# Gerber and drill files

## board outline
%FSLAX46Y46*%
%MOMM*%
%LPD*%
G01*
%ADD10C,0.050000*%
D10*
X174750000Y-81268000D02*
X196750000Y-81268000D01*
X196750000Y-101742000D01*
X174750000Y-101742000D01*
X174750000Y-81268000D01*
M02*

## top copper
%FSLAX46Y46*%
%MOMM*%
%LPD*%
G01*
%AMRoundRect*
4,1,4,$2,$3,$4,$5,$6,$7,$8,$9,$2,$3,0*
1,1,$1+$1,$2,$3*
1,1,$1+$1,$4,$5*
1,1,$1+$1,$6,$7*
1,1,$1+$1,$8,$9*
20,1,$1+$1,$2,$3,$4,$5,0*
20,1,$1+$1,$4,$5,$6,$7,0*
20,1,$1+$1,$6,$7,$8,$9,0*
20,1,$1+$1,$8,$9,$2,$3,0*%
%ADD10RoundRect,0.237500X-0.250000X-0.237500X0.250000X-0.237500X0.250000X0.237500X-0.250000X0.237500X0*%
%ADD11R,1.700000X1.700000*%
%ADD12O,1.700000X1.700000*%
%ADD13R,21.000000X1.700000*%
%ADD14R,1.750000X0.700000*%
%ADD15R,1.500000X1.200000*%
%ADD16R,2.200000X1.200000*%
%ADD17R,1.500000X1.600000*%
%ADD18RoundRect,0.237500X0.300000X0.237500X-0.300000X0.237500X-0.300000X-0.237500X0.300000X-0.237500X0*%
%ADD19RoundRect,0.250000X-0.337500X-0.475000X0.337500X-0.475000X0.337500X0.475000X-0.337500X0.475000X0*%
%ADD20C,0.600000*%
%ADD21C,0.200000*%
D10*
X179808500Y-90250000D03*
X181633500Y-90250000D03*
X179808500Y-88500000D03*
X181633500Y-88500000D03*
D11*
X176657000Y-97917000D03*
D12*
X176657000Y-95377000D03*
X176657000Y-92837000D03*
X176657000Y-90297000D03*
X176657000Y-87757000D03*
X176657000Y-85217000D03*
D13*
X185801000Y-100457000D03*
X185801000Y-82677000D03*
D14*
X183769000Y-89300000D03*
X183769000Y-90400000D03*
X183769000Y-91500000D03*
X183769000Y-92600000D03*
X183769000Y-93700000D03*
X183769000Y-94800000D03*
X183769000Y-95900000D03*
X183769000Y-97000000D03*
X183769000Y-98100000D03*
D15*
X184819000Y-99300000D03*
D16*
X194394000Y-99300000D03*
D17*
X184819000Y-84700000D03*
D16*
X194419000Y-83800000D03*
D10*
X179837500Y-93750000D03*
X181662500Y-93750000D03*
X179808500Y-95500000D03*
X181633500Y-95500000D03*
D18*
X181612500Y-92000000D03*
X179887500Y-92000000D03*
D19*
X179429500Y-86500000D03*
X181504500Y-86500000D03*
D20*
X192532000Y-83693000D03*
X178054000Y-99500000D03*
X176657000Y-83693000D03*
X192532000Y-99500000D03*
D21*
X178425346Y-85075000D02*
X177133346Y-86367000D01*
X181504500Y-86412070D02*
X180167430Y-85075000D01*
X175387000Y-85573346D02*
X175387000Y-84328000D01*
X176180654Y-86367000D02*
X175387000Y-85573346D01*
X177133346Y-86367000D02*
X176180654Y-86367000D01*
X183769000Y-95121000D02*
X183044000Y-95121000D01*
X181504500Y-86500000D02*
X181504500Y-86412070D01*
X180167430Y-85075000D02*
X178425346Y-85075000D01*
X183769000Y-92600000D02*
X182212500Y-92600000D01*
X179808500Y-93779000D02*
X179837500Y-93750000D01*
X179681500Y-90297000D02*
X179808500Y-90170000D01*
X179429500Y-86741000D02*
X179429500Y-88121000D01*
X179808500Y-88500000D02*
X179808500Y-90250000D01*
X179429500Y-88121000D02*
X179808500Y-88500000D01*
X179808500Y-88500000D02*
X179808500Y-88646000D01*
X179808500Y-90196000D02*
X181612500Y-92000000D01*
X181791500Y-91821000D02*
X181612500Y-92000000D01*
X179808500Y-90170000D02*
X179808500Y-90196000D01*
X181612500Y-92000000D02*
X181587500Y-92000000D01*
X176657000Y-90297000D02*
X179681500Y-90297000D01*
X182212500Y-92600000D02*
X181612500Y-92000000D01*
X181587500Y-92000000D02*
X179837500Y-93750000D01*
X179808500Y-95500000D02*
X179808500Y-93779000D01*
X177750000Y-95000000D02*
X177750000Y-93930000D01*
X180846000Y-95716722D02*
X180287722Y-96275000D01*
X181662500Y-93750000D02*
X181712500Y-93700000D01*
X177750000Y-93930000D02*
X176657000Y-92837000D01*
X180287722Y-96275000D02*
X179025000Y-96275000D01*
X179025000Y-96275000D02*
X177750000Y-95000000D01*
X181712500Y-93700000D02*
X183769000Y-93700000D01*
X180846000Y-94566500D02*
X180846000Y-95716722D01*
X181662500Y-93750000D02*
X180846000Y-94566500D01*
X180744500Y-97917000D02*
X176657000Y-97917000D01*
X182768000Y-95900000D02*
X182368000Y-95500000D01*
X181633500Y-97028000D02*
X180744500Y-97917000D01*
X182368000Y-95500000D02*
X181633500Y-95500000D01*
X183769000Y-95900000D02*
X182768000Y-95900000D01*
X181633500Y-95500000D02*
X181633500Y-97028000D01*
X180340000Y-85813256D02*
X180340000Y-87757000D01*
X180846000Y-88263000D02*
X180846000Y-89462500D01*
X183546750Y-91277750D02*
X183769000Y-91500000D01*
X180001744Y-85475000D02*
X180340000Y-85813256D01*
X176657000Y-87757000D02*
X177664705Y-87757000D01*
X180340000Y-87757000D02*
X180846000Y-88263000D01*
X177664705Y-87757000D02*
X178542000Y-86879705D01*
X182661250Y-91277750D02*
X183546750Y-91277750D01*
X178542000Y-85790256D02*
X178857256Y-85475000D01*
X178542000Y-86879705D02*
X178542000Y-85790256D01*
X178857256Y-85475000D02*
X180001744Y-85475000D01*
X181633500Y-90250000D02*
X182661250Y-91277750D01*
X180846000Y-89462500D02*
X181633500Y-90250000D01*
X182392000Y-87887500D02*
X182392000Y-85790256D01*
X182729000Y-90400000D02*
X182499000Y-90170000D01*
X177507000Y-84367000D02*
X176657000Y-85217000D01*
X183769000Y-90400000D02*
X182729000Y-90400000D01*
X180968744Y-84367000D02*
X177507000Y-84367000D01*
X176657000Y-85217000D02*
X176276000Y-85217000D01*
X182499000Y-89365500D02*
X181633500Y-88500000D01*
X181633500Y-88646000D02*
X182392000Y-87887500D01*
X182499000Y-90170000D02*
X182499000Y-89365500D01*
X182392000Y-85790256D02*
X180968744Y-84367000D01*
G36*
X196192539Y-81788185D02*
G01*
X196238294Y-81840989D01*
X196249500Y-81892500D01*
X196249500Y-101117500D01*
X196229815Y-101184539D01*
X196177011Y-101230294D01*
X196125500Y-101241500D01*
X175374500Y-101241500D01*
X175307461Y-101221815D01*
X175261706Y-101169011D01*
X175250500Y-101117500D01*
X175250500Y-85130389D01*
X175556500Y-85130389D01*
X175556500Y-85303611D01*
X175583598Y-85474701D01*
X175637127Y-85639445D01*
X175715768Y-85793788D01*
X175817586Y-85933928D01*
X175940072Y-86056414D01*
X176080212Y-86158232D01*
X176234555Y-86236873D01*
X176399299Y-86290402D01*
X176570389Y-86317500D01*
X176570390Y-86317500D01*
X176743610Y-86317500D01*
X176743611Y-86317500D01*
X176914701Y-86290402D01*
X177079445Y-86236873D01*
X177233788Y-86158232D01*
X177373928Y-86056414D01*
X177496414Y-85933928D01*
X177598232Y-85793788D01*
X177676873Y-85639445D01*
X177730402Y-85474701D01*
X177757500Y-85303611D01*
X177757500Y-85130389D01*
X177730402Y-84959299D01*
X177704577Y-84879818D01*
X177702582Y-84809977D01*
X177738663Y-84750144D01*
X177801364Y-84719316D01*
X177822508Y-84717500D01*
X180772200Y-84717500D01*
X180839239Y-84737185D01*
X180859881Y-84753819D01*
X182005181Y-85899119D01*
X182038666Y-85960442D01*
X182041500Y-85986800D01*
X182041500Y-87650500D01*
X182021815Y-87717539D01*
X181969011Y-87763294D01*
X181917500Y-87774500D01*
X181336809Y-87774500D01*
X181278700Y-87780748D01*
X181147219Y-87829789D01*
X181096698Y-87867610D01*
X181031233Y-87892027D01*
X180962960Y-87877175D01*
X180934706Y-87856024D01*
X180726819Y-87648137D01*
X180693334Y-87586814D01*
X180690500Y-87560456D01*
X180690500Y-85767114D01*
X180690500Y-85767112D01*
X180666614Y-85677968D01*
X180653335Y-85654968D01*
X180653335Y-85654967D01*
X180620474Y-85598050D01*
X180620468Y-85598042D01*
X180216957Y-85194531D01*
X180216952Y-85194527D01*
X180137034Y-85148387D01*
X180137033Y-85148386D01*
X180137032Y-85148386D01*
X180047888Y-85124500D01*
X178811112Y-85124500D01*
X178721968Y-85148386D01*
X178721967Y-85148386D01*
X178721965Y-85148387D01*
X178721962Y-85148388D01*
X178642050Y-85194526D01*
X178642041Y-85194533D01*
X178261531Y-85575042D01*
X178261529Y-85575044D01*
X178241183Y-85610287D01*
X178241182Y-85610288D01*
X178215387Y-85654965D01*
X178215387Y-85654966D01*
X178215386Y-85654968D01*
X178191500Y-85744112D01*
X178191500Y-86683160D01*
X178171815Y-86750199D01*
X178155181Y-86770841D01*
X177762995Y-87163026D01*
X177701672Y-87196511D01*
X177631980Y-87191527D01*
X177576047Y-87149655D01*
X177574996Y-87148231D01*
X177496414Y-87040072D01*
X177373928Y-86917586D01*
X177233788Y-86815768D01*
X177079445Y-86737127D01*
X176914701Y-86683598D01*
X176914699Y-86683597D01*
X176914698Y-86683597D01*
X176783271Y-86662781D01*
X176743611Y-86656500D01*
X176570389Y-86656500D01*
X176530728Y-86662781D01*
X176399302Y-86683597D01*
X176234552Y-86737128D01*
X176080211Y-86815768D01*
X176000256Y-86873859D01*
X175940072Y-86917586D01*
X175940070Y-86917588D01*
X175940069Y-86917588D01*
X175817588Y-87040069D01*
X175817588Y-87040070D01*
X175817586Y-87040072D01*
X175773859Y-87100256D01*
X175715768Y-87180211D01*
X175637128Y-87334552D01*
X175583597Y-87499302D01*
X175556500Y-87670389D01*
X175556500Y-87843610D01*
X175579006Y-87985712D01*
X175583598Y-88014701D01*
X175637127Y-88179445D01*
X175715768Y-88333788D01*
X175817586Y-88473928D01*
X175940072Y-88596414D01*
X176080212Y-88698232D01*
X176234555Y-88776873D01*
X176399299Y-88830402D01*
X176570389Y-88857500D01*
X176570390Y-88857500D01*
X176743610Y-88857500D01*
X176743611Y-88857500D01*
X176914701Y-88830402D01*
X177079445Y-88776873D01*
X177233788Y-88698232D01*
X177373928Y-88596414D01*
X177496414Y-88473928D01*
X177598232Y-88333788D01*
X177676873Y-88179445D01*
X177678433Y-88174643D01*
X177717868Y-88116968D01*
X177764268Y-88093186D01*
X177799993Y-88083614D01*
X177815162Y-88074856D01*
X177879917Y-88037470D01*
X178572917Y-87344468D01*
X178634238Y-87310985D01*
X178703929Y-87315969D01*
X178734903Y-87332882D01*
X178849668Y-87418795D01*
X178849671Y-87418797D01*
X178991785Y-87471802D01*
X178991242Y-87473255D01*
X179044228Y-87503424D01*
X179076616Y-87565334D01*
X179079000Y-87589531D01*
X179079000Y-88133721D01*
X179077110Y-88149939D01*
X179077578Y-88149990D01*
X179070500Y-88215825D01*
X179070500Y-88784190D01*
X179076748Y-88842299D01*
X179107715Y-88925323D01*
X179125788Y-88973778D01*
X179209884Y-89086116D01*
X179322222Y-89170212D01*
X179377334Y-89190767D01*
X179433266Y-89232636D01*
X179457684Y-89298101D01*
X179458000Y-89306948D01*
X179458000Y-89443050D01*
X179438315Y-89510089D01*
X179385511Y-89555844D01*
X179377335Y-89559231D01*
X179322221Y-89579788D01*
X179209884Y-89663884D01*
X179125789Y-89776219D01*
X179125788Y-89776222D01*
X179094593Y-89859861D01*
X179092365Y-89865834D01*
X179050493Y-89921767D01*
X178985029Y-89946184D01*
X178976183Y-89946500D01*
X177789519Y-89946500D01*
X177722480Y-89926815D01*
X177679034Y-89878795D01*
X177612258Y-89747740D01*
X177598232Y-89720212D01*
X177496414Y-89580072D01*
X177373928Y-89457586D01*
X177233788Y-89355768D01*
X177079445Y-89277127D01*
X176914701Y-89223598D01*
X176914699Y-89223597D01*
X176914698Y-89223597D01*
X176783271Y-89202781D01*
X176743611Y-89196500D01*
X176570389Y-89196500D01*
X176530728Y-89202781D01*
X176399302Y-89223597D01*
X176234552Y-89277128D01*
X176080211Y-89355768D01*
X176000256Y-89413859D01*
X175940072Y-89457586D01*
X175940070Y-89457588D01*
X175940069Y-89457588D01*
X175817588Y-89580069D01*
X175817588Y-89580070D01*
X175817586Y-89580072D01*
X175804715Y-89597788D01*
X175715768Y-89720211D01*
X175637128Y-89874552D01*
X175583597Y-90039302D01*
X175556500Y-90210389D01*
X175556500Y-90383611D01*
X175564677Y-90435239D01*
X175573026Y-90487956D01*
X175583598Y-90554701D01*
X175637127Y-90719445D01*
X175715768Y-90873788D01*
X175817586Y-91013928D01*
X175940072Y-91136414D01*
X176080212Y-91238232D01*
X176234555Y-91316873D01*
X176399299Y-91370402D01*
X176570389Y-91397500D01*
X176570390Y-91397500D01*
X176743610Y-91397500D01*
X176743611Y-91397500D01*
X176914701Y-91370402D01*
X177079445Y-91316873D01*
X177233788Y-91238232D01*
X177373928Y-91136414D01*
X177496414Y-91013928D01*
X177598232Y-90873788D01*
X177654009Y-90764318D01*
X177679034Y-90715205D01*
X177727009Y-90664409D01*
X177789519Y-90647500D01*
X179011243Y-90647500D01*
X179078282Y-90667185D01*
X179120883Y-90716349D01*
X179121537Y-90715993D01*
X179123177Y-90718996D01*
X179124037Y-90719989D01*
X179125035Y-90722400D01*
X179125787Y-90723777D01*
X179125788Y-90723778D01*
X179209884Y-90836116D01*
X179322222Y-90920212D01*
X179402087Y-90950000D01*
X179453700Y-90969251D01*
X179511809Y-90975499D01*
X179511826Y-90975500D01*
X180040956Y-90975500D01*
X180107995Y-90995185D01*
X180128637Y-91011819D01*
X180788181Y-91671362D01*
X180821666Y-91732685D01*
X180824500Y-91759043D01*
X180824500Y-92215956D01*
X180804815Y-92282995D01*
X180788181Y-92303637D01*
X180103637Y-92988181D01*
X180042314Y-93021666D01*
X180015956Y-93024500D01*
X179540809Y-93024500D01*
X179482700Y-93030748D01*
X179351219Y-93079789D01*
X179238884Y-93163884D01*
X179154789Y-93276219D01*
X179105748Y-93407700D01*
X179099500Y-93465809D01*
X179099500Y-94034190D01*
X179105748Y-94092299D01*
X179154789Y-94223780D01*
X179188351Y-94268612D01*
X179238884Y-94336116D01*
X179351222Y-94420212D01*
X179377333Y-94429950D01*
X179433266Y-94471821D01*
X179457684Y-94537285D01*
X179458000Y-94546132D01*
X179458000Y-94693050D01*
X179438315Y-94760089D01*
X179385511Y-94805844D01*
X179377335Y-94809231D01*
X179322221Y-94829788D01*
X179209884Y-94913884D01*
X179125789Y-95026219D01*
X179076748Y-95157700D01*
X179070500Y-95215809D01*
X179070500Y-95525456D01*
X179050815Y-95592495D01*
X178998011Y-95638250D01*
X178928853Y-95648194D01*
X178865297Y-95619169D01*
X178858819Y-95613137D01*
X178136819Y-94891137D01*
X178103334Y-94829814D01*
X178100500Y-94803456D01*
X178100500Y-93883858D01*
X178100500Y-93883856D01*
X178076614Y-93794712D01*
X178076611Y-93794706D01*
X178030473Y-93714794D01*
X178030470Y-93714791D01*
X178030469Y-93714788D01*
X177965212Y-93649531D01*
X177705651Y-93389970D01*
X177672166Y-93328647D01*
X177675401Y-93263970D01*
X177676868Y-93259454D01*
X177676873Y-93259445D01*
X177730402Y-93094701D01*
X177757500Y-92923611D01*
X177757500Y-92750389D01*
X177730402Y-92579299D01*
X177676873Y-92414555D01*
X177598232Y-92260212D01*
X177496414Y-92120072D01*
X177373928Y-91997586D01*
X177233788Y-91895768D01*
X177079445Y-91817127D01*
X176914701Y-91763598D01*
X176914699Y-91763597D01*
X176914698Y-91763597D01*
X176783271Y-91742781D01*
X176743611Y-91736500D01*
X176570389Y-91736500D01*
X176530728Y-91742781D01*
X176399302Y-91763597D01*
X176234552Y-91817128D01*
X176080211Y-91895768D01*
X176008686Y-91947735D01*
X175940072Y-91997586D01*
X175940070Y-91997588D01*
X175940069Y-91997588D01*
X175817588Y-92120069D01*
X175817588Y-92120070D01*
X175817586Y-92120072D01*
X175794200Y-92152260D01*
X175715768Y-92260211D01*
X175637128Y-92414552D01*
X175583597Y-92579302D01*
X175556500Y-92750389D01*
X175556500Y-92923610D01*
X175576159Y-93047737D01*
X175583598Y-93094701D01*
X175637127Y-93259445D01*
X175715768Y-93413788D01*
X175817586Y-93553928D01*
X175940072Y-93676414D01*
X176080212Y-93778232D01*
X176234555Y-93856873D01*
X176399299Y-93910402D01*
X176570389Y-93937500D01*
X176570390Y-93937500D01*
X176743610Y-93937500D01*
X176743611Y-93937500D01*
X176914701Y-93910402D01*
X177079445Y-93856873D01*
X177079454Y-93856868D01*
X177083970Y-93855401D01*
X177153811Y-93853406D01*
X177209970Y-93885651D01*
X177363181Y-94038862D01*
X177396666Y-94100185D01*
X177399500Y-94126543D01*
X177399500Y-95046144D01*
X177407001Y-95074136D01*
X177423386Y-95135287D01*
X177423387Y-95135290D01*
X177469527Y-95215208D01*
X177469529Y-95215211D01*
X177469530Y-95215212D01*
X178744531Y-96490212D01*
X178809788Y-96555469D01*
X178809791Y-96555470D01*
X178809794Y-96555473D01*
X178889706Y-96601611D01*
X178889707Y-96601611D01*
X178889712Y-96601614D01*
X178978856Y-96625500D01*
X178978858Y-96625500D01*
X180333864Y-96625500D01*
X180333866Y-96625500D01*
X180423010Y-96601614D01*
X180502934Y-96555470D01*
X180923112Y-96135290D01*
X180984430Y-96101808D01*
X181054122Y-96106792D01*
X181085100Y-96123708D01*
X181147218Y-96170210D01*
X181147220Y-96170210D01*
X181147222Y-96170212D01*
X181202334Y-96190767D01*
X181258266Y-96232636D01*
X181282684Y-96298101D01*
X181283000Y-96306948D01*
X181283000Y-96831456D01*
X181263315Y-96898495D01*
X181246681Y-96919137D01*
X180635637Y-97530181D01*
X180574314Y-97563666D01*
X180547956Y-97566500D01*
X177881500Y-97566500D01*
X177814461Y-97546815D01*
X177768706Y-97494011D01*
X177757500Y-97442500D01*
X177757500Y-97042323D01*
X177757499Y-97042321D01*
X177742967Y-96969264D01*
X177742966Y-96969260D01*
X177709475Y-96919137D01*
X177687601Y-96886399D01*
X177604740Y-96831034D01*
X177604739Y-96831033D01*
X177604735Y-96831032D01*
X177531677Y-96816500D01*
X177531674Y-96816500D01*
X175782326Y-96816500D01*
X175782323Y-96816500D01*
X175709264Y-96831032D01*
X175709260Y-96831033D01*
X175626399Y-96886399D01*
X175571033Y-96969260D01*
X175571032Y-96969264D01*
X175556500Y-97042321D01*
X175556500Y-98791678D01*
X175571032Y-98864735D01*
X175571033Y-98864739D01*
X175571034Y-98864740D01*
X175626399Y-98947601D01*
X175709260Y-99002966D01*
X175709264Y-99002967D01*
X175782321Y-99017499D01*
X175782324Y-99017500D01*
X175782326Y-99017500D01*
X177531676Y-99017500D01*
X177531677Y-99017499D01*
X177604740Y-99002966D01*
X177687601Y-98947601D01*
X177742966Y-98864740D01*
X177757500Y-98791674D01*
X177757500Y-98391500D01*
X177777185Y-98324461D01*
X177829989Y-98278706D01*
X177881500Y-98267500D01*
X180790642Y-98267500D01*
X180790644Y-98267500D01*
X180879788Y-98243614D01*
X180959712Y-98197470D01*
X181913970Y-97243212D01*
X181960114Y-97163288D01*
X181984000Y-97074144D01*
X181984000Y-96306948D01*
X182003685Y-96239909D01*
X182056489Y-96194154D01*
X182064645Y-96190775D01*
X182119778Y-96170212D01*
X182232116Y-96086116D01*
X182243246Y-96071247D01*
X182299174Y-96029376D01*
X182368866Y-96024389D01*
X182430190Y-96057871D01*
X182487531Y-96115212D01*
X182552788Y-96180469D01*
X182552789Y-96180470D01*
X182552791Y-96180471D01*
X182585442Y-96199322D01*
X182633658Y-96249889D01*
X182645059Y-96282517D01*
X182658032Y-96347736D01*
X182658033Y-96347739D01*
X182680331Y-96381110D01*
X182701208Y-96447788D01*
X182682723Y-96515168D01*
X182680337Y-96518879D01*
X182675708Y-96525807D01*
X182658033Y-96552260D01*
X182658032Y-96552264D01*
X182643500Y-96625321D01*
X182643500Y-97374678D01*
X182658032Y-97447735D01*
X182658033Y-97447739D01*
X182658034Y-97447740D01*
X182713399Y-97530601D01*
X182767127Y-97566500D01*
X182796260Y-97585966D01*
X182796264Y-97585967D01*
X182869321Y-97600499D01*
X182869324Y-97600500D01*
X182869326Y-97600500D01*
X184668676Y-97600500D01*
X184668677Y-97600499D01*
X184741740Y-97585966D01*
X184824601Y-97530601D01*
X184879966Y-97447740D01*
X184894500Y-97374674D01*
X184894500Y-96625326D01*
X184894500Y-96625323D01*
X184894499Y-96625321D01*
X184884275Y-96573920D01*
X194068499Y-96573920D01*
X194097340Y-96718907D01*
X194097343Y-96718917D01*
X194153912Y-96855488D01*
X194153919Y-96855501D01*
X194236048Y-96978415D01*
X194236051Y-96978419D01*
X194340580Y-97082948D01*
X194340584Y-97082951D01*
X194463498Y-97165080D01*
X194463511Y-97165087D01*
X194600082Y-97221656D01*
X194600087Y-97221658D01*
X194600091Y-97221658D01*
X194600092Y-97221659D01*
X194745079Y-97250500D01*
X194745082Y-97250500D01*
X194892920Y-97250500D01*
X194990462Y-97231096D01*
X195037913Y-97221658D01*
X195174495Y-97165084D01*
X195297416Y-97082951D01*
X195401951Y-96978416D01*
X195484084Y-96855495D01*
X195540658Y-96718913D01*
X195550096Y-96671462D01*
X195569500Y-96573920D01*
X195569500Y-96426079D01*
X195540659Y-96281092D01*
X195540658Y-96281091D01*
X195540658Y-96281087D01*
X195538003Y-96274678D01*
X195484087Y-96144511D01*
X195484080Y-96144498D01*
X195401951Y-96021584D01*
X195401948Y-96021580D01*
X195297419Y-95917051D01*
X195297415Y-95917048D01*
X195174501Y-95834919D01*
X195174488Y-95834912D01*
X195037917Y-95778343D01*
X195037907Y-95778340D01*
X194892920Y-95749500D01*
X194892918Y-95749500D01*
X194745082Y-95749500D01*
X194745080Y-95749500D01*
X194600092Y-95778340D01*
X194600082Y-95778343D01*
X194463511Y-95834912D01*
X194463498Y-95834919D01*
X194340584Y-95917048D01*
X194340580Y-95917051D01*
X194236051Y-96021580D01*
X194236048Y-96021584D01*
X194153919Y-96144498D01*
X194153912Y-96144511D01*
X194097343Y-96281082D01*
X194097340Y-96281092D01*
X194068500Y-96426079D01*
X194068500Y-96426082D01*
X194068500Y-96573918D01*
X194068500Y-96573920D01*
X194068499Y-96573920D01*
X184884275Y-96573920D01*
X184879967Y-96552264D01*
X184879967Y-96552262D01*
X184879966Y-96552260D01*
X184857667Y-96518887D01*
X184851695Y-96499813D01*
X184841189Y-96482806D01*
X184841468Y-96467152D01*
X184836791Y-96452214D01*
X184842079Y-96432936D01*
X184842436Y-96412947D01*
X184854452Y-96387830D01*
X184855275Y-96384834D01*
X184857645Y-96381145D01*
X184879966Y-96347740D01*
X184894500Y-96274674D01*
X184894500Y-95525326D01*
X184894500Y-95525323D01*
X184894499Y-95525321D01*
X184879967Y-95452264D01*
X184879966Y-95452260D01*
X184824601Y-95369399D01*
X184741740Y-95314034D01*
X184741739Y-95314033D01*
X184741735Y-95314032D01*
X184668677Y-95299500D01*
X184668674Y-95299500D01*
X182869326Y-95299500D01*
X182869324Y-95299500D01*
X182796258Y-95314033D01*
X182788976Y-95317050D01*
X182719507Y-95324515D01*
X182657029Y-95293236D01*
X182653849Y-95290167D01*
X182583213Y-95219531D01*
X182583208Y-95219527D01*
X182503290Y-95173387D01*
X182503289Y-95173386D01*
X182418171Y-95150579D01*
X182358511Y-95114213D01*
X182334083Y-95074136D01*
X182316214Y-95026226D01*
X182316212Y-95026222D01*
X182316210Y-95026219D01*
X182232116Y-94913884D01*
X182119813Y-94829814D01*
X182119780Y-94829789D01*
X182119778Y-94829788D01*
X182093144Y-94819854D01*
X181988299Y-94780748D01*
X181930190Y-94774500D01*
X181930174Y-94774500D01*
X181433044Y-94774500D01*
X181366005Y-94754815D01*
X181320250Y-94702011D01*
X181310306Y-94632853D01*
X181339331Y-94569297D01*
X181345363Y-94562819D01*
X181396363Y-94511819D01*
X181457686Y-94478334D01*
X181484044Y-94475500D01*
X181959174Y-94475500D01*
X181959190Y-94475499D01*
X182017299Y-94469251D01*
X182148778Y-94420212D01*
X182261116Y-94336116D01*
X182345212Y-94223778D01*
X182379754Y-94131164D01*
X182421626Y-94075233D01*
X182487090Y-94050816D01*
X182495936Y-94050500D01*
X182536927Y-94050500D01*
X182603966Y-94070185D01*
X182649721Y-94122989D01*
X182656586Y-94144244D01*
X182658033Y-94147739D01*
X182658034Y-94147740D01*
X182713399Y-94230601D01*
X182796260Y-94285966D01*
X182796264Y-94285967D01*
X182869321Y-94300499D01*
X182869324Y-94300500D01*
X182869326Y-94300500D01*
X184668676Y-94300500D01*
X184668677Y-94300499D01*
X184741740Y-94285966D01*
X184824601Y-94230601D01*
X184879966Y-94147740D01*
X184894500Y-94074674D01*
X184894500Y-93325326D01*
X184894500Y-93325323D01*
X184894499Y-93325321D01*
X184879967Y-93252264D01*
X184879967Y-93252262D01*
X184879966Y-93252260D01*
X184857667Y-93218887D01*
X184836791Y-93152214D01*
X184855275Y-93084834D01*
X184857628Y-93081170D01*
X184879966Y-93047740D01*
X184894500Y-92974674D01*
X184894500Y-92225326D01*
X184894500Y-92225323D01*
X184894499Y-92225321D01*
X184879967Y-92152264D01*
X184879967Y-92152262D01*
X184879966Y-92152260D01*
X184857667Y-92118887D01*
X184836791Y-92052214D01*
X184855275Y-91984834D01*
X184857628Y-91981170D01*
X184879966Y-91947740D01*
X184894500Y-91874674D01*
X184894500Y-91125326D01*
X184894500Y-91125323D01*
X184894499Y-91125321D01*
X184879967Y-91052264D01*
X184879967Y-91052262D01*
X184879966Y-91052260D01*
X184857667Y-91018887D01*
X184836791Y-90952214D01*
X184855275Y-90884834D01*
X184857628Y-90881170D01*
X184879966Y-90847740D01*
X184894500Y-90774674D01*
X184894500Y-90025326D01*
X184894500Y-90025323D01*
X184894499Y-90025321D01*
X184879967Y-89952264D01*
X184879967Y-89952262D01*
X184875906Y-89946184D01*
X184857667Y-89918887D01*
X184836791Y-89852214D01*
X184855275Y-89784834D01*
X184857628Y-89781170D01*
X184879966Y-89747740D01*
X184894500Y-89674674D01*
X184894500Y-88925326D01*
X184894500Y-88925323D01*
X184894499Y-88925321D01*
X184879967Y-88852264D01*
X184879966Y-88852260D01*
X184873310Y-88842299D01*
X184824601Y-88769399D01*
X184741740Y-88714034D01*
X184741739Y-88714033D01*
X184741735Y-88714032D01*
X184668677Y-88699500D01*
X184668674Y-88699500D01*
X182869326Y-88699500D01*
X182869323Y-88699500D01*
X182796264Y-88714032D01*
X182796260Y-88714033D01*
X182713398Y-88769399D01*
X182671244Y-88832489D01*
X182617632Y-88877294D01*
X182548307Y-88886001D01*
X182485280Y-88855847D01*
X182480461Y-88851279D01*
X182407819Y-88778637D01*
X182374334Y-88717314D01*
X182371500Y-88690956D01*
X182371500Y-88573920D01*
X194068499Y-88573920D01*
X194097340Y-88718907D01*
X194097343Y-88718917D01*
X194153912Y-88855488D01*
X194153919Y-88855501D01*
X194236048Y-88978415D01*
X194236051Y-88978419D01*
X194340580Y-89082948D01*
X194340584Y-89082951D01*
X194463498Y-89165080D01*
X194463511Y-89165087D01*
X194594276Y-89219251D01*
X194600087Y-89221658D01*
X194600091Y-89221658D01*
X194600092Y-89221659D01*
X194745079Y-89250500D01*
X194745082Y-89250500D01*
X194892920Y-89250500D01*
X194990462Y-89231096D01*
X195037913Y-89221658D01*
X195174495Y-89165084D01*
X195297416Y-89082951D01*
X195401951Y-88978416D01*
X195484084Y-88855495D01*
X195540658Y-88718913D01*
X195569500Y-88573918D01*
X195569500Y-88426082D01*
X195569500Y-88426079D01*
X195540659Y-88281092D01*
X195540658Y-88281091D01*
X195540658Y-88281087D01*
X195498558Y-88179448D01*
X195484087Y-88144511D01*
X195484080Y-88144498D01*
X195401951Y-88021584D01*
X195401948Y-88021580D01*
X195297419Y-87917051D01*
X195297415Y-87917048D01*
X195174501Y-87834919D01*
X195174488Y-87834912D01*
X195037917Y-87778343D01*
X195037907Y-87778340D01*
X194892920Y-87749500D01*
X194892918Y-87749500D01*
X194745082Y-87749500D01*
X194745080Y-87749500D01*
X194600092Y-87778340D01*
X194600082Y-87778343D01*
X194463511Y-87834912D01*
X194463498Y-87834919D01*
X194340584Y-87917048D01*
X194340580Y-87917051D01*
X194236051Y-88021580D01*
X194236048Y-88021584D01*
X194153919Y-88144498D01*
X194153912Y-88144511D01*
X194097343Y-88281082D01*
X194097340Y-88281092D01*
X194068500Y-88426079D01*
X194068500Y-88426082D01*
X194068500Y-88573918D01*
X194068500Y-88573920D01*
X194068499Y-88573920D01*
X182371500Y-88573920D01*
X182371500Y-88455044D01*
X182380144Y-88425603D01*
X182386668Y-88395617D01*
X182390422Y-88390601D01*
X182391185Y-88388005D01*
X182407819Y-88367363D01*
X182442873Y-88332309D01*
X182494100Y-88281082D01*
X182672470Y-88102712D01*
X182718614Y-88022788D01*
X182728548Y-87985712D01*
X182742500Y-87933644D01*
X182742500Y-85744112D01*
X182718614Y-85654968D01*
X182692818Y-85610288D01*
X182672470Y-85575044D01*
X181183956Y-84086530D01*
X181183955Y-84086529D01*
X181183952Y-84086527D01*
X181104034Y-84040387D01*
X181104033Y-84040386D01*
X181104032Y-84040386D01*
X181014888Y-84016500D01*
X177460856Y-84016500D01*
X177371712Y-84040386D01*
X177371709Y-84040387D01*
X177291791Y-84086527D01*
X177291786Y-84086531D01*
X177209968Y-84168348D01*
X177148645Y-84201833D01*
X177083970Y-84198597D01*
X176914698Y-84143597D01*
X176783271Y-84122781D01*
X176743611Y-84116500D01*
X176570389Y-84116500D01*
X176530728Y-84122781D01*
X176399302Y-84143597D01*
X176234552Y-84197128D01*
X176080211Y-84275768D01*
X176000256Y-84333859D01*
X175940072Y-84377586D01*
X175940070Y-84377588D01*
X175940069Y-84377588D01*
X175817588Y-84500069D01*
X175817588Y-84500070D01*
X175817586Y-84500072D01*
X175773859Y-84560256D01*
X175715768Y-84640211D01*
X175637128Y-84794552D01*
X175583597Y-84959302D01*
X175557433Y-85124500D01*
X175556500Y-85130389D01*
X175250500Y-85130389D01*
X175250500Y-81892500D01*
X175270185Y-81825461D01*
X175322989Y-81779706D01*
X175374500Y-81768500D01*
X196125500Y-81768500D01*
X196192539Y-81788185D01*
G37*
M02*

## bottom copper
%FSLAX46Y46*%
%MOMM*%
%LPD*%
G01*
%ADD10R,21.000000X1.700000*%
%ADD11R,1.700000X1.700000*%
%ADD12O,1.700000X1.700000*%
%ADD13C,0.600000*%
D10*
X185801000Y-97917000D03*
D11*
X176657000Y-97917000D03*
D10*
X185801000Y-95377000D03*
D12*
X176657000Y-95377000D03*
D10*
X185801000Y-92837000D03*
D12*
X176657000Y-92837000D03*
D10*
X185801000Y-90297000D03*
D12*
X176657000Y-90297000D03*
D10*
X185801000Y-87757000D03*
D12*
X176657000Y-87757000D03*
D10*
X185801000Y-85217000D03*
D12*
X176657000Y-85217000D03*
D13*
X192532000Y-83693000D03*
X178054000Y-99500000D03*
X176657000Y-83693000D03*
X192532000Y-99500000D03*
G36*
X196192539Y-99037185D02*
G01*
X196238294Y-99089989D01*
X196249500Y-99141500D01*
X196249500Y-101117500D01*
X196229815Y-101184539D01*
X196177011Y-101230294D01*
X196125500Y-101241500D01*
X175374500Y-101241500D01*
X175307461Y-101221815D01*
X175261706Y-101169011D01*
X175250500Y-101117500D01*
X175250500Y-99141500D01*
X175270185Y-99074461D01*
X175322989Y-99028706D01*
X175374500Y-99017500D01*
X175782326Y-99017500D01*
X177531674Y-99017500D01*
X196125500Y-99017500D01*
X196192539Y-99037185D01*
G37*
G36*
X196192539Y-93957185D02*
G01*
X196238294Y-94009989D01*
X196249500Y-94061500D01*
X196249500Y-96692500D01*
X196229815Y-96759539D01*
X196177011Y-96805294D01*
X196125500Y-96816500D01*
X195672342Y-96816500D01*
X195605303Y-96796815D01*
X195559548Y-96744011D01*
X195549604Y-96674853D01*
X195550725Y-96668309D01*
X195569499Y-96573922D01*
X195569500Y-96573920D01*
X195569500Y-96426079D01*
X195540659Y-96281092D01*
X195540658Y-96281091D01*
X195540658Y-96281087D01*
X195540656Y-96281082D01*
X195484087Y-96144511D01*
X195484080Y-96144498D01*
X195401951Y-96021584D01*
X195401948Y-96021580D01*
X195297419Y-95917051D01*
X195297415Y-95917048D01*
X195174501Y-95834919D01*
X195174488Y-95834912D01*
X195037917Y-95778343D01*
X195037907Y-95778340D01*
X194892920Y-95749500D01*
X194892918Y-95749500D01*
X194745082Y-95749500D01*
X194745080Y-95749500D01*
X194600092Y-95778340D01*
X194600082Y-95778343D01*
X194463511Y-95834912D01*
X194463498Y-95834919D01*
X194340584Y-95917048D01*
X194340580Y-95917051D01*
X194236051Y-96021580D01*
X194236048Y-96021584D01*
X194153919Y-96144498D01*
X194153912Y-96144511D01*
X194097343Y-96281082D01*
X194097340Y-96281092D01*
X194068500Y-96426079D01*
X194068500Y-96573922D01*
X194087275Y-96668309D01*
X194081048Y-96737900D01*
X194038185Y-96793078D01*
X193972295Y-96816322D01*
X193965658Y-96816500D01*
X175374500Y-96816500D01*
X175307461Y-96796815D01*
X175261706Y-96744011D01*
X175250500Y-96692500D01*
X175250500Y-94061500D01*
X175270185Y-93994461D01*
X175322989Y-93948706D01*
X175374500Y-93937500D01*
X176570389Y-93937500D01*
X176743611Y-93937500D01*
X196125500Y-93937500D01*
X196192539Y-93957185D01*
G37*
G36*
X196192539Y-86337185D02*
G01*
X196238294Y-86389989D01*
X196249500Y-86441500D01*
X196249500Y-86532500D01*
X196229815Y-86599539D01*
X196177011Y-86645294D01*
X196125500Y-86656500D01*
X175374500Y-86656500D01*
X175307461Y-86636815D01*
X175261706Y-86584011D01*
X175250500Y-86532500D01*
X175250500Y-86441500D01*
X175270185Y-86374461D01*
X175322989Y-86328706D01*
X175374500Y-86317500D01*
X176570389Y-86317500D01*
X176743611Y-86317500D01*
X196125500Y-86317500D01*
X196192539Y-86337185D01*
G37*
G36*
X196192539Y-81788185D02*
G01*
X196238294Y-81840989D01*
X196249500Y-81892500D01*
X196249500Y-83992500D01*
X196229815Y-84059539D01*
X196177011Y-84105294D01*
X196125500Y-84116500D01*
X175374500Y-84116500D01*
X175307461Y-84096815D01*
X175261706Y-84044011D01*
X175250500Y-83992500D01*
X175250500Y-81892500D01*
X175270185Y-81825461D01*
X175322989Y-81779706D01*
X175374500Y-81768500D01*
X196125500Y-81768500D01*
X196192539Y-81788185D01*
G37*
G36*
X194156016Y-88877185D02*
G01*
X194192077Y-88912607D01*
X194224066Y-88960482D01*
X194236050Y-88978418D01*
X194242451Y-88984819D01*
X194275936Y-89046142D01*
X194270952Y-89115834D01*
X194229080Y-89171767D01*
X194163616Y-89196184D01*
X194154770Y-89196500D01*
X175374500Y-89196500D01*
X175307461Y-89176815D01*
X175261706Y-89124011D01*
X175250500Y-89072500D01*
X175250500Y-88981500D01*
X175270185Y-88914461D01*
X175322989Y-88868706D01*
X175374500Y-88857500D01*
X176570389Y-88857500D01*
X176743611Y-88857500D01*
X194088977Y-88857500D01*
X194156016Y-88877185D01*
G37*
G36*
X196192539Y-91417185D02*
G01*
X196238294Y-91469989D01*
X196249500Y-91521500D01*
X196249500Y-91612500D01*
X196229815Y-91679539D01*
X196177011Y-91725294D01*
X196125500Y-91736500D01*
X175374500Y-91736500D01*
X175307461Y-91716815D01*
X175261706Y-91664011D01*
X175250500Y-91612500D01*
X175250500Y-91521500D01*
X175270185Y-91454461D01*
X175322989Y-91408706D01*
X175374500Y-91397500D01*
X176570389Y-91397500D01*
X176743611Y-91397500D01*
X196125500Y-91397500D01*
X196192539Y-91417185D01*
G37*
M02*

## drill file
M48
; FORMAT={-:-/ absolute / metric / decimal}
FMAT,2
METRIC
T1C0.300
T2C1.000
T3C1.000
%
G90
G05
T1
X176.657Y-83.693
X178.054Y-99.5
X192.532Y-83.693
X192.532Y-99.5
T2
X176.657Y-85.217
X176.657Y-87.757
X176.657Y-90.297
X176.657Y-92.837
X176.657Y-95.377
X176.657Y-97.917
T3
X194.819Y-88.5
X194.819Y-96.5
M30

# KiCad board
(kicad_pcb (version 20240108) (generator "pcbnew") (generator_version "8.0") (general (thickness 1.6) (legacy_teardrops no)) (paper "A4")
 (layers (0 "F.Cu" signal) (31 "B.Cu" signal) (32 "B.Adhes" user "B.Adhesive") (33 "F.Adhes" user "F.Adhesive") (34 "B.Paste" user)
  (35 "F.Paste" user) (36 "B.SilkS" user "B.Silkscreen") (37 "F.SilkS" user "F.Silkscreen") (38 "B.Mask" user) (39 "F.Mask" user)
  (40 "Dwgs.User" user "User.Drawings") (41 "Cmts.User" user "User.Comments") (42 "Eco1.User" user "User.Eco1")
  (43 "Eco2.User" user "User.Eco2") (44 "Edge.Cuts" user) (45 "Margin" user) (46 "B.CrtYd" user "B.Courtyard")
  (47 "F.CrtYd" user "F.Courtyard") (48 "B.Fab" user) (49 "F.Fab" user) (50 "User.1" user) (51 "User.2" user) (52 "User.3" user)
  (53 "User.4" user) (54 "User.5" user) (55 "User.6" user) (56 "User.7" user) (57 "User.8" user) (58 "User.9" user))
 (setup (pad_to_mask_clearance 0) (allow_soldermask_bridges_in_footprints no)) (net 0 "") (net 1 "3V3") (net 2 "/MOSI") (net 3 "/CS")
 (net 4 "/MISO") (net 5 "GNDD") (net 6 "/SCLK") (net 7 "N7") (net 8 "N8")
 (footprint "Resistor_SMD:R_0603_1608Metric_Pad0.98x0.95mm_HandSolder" (layer "F.Cu") (at 180.721 90.25)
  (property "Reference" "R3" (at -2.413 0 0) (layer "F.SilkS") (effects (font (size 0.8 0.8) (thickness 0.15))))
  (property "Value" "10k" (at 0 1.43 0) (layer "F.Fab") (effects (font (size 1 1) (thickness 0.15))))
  (pad "1" smd roundrect (at -0.9125 0) (size 0.975 0.95) (layers "F.Cu" "F.Paste" "F.Mask") (roundrect_rratio 0.25) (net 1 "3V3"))
  (pad "2" smd roundrect (at 0.9125 0) (size 0.975 0.95) (layers "F.Cu" "F.Paste" "F.Mask") (roundrect_rratio 0.25) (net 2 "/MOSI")))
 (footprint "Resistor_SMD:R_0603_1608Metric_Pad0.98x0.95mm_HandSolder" (layer "F.Cu") (at 180.721 88.5)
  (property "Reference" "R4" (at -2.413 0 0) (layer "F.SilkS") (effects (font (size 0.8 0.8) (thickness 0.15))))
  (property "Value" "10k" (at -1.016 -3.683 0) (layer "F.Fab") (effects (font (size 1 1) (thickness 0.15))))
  (pad "1" smd roundrect (at -0.9125 0) (size 0.975 0.95) (layers "F.Cu" "F.Paste" "F.Mask") (roundrect_rratio 0.25) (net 1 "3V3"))
  (pad "2" smd roundrect (at 0.9125 0) (size 0.975 0.95) (layers "F.Cu" "F.Paste" "F.Mask") (roundrect_rratio 0.25) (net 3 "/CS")))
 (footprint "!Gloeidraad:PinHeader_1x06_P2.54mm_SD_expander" (layer "F.Cu") (at 176.657 97.917 180)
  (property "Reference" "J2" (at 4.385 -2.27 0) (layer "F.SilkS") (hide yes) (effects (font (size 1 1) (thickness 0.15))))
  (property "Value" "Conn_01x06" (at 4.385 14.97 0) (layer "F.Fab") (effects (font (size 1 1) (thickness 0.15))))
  (pad "1" smd rect (at -9.144 0 180) (size 21 1.7) (layers "B.Cu" "B.Paste" "B.Mask") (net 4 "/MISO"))
  (pad "1" thru_hole rect (at 0 0 180) (size 1.7 1.7) (drill 1) (layers "*.Cu" "*.Mask") (remove_unused_layers no) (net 4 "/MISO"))
  (pad "2" smd rect (at -9.144 2.54 180) (size 21 1.7) (layers "B.Cu" "B.Paste" "B.Mask") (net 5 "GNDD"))
  (pad "2" thru_hole oval (at 0 2.54 180) (size 1.7 1.7) (drill 1) (layers "*.Cu" "*.Mask") (remove_unused_layers no) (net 5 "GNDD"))
  (pad "3" smd rect (at -9.144 5.08 180) (size 21 1.7) (layers "B.Cu" "B.Paste" "B.Mask") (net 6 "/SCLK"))
  (pad "3" thru_hole oval (at 0 5.08 180) (size 1.7 1.7) (drill 1) (layers "*.Cu" "*.Mask") (remove_unused_layers no) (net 6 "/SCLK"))
  (pad "4" smd rect (at -9.144 7.62 180) (size 21 1.7) (layers "B.Cu" "B.Paste" "B.Mask") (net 1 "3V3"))
  (pad "4" thru_hole oval (at 0 7.62 180) (size 1.7 1.7) (drill 1) (layers "*.Cu" "*.Mask") (remove_unused_layers no) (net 1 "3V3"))
  (pad "5" smd rect (at -9.144 10.16 180) (size 21 1.7) (layers "B.Cu" "B.Paste" "B.Mask") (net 2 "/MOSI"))
  (pad "5" thru_hole oval (at 0 10.16 180) (size 1.7 1.7) (drill 1) (layers "*.Cu" "*.Mask") (remove_unused_layers no) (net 2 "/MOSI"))
  (pad "6" smd rect (at -9.144 12.7 180) (size 21 1.7) (layers "B.Cu" "B.Paste" "B.Mask") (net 3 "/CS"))
  (pad "6" thru_hole oval (at 0 12.7 180) (size 1.7 1.7) (drill 1) (layers "*.Cu" "*.Mask") (remove_unused_layers no) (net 3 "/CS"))
  (pad "10" smd rect (at -9.144 -2.54 180) (size 21 1.7) (layers "F.Cu" "F.Paste" "F.Mask") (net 5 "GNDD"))
  (pad "10" smd rect (at -9.144 15.24 180) (size 21 1.7) (layers "F.Cu" "F.Paste" "F.Mask") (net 5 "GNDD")))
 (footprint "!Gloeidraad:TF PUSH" (layer "F.Cu") (at 194.819 96.5 90)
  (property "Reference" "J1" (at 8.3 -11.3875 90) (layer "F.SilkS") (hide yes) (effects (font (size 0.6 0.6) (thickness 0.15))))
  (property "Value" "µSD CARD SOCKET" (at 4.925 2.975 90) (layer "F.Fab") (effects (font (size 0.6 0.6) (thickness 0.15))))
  (pad "" np_thru_hole circle (at 0 0 90) (size 0.7 0.7) (drill 1) (layers "F&B.Cu" "*.Mask"))
  (pad "" np_thru_hole circle (at 8 0 90) (size 0.7 0.7) (drill 1) (layers "F&B.Cu" "*.Mask"))
  (pad "1" smd rect (at 7.2 -11.05 90) (size 0.7 1.75) (layers "F.Cu" "F.Paste" "F.Mask") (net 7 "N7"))
  (pad "2" smd rect (at 6.1 -11.05 90) (size 0.7 1.75) (layers "F.Cu" "F.Paste" "F.Mask") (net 3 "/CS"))
  (pad "3" smd rect (at 5 -11.05 90) (size 0.7 1.75) (layers "F.Cu" "F.Paste" "F.Mask") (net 2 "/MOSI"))
  (pad "4" smd rect (at 3.9 -11.05 90) (size 0.7 1.75) (layers "F.Cu" "F.Paste" "F.Mask") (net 1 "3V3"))
  (pad "5" smd rect (at 2.8 -11.05 90) (size 0.7 1.75) (layers "F.Cu" "F.Paste" "F.Mask") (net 6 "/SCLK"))
  (pad "6" smd rect (at 1.7 -11.05 90) (size 0.7 1.75) (layers "F.Cu" "F.Paste" "F.Mask") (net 5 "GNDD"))
  (pad "7" smd rect (at 0.6 -11.05 90) (size 0.7 1.75) (layers "F.Cu" "F.Paste" "F.Mask") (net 4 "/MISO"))
  (pad "8" smd rect (at -0.5 -11.05 90) (size 0.7 1.75) (layers "F.Cu" "F.Paste" "F.Mask") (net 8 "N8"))
  (pad "9" smd rect (at -1.6 -11.05 90) (size 0.7 1.75) (layers "F.Cu" "F.Paste" "F.Mask") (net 5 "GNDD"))
  (pad "10" smd rect (at -2.8 -10 90) (size 1.2 1.5) (layers "F.Cu" "F.Paste" "F.Mask") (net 5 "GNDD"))
  (pad "10" smd rect (at -2.8 -0.425 90) (size 1.2 2.2) (layers "F.Cu" "F.Paste" "F.Mask") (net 5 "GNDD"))
  (pad "10" smd rect (at 11.8 -10 90) (size 1.6 1.5) (layers "F.Cu" "F.Paste" "F.Mask") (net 5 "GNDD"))
  (pad "10" smd rect (at 12.7 -0.4 90) (size 1.2 2.2) (layers "F.Cu" "F.Paste" "F.Mask") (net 5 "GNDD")))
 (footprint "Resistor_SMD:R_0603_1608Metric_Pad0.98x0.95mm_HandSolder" (layer "F.Cu") (at 180.75 93.75)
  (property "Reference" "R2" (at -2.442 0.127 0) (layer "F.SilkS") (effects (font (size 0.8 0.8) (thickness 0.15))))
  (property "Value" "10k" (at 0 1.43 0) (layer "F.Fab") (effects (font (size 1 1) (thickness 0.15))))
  (pad "1" smd roundrect (at -0.9125 0) (size 0.975 0.95) (layers "F.Cu" "F.Paste" "F.Mask") (roundrect_rratio 0.25) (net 1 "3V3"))
  (pad "2" smd roundrect (at 0.9125 0) (size 0.975 0.95) (layers "F.Cu" "F.Paste" "F.Mask") (roundrect_rratio 0.25) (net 6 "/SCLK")))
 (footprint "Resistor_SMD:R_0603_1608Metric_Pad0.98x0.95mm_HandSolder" (layer "F.Cu") (at 180.721 95.5)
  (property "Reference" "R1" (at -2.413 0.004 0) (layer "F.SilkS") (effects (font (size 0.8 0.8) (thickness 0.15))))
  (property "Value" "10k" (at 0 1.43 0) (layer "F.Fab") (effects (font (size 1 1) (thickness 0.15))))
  (pad "1" smd roundrect (at -0.9125 0) (size 0.975 0.95) (layers "F.Cu" "F.Paste" "F.Mask") (roundrect_rratio 0.25) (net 1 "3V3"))
  (pad "2" smd roundrect (at 0.9125 0) (size 0.975 0.95) (layers "F.Cu" "F.Paste" "F.Mask") (roundrect_rratio 0.25) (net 4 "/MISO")))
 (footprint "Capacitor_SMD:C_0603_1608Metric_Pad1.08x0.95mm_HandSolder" (layer "F.Cu") (at 180.75 92 180)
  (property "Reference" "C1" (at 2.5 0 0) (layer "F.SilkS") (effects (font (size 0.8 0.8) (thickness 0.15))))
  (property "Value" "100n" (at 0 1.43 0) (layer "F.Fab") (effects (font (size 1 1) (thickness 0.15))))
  (pad "1" smd roundrect (at -0.8625 0 180) (size 1.075 0.95) (layers "F.Cu" "F.Paste" "F.Mask") (roundrect_rratio 0.25) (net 1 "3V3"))
  (pad "2" smd roundrect (at 0.8625 0 180) (size 1.075 0.95) (layers "F.Cu" "F.Paste" "F.Mask") (roundrect_rratio 0.25) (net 5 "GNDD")))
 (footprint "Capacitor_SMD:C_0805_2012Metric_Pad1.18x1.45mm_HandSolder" (layer "F.Cu") (at 180.467 86.5)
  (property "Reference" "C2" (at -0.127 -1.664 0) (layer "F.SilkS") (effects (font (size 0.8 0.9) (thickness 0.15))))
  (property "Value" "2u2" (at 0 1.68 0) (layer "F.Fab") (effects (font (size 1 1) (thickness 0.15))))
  (pad "1" smd roundrect (at -1.0375 0) (size 1.175 1.45) (layers "F.Cu" "F.Paste" "F.Mask") (roundrect_rratio 0.212766) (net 1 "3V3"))
  (pad "2" smd roundrect (at 1.0375 0) (size 1.175 1.45) (layers "F.Cu" "F.Paste" "F.Mask") (roundrect_rratio 0.212766) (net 5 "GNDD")))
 (gr_rect (start 174.75 81.268) (end 196.75 101.742) (stroke (width 0.05) (type default)) (fill none) (layer "Edge.Cuts"))
 (segment (start 178.425346 85.075) (end 177.133346 86.367) (width 0.2) (layer "F.Cu") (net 5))
 (segment (start 181.5045 86.41207) (end 180.16743 85.075) (width 0.2) (layer "F.Cu") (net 5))
 (segment (start 175.387 85.573346) (end 175.387 84.328) (width 0.2) (layer "F.Cu") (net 5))
 (segment (start 176.180654 86.367) (end 175.387 85.573346) (width 0.2) (layer "F.Cu") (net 5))
 (segment (start 177.133346 86.367) (end 176.180654 86.367) (width 0.2) (layer "F.Cu") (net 5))
 (segment (start 183.769 95.121) (end 183.044 95.121) (width 0.2) (layer "F.Cu") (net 5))
 (segment (start 181.5045 86.5) (end 181.5045 86.41207) (width 0.2) (layer "F.Cu") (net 5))
 (segment (start 180.16743 85.075) (end 178.425346 85.075) (width 0.2) (layer "F.Cu") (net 5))
 (via (at 192.532 83.693) (size 0.6) (drill 0.3) (layers "F.Cu" "B.Cu") (free yes) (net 5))
 (via (at 178.054 99.5) (size 0.6) (drill 0.3) (layers "F.Cu" "B.Cu") (free yes) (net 5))
 (via (at 176.657 83.693) (size 0.6) (drill 0.3) (layers "F.Cu" "B.Cu") (free yes) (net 5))
 (via (at 192.532 99.5) (size 0.6) (drill 0.3) (layers "F.Cu" "B.Cu") (free yes) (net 5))
 (segment (start 183.769 92.6) (end 182.2125 92.6) (width 0.2) (layer "F.Cu") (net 1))
 (segment (start 179.8085 93.779) (end 179.8375 93.75) (width 0.2) (layer "F.Cu") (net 1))
 (segment (start 179.6815 90.297) (end 179.8085 90.17) (width 0.2) (layer "F.Cu") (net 1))
 (segment (start 179.4295 86.741) (end 179.4295 88.121) (width 0.2) (layer "F.Cu") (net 1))
 (segment (start 179.8085 88.5) (end 179.8085 90.25) (width 0.2) (layer "F.Cu") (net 1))
 (segment (start 179.4295 88.121) (end 179.8085 88.5) (width 0.2) (layer "F.Cu") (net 1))
 (segment (start 179.8085 88.5) (end 179.8085 88.646) (width 0.2) (layer "F.Cu") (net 1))
 (segment (start 179.8085 90.196) (end 181.6125 92) (width 0.2) (layer "F.Cu") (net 1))
 (segment (start 181.7915 91.821) (end 181.6125 92) (width 0.2) (layer "F.Cu") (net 1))
 (segment (start 179.8085 90.17) (end 179.8085 90.196) (width 0.2) (layer "F.Cu") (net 1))
 (segment (start 181.6125 92) (end 181.5875 92) (width 0.2) (layer "F.Cu") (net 1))
 (segment (start 176.657 90.297) (end 179.6815 90.297) (width 0.2) (layer "F.Cu") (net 1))
 (segment (start 182.2125 92.6) (end 181.6125 92) (width 0.2) (layer "F.Cu") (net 1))
 (segment (start 181.5875 92) (end 179.8375 93.75) (width 0.2) (layer "F.Cu") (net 1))
 (segment (start 179.8085 95.5) (end 179.8085 93.779) (width 0.2) (layer "F.Cu") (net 1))
 (segment (start 177.75 95) (end 177.75 93.93) (width 0.2) (layer "F.Cu") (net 6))
 (segment (start 180.846 95.716722) (end 180.287722 96.275) (width 0.2) (layer "F.Cu") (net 6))
 (segment (start 181.6625 93.75) (end 181.7125 93.7) (width 0.2) (layer "F.Cu") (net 6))
 (segment (start 177.75 93.93) (end 176.657 92.837) (width 0.2) (layer "F.Cu") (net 6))
 (segment (start 180.287722 96.275) (end 179.025 96.275) (width 0.2) (layer "F.Cu") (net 6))
 (segment (start 179.025 96.275) (end 177.75 95) (width 0.2) (layer "F.Cu") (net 6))
 (segment (start 181.7125 93.7) (end 183.769 93.7) (width 0.2) (layer "F.Cu") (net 6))
 (segment (start 180.846 94.5665) (end 180.846 95.716722) (width 0.2) (layer "F.Cu") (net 6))
 (segment (start 181.6625 93.75) (end 180.846 94.5665) (width 0.2) (layer "F.Cu") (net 6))
 (segment (start 180.7445 97.917) (end 176.657 97.917) (width 0.2) (layer "F.Cu") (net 4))
 (segment (start 182.768 95.9) (end 182.368 95.5) (width 0.2) (layer "F.Cu") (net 4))
 (segment (start 181.6335 97.028) (end 180.7445 97.917) (width 0.2) (layer "F.Cu") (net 4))
 (segment (start 182.368 95.5) (end 181.6335 95.5) (width 0.2) (layer "F.Cu") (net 4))
 (segment (start 183.769 95.9) (end 182.768 95.9) (width 0.2) (layer "F.Cu") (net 4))
 (segment (start 181.6335 95.5) (end 181.6335 97.028) (width 0.2) (layer "F.Cu") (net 4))
 (segment (start 180.34 85.813256) (end 180.34 87.757) (width 0.2) (layer "F.Cu") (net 2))
 (segment (start 180.846 88.263) (end 180.846 89.4625) (width 0.2) (layer "F.Cu") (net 2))
 (segment (start 183.54675 91.27775) (end 183.769 91.5) (width 0.2) (layer "F.Cu") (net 2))
 (segment (start 180.001744 85.475) (end 180.34 85.813256) (width 0.2) (layer "F.Cu") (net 2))
 (segment (start 176.657 87.757) (end 177.664705 87.757) (width 0.2) (layer "F.Cu") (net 2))
 (segment (start 180.34 87.757) (end 180.846 88.263) (width 0.2) (layer "F.Cu") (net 2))
 (segment (start 177.664705 87.757) (end 178.542 86.879705) (width 0.2) (layer "F.Cu") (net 2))
 (segment (start 182.66125 91.27775) (end 183.54675 91.27775) (width 0.2) (layer "F.Cu") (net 2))
 (segment (start 178.542 85.790256) (end 178.857256 85.475) (width 0.2) (layer "F.Cu") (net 2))
 (segment (start 178.542 86.879705) (end 178.542 85.790256) (width 0.2) (layer "F.Cu") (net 2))
 (segment (start 178.857256 85.475) (end 180.001744 85.475) (width 0.2) (layer "F.Cu") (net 2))
 (segment (start 181.6335 90.25) (end 182.66125 91.27775) (width 0.2) (layer "F.Cu") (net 2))
 (segment (start 180.846 89.4625) (end 181.6335 90.25) (width 0.2) (layer "F.Cu") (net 2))
 (segment (start 182.392 87.8875) (end 182.392 85.790256) (width 0.2) (layer "F.Cu") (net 3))
 (segment (start 182.729 90.4) (end 182.499 90.17) (width 0.2) (layer "F.Cu") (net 3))
 (segment (start 177.507 84.367) (end 176.657 85.217) (width 0.2) (layer "F.Cu") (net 3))
 (segment (start 183.769 90.4) (end 182.729 90.4) (width 0.2) (layer "F.Cu") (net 3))
 (segment (start 180.968744 84.367) (end 177.507 84.367) (width 0.2) (layer "F.Cu") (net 3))
 (segment (start 176.657 85.217) (end 176.276 85.217) (width 0.2) (layer "F.Cu") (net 3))
 (segment (start 182.499 89.3655) (end 181.6335 88.5) (width 0.2) (layer "F.Cu") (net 3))
 (segment (start 181.6335 88.646) (end 182.392 87.8875) (width 0.2) (layer "F.Cu") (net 3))
 (segment (start 182.499 90.17) (end 182.499 89.3655) (width 0.2) (layer "F.Cu") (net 3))
 (segment (start 182.392 85.790256) (end 180.968744 84.367) (width 0.2) (layer "F.Cu") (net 3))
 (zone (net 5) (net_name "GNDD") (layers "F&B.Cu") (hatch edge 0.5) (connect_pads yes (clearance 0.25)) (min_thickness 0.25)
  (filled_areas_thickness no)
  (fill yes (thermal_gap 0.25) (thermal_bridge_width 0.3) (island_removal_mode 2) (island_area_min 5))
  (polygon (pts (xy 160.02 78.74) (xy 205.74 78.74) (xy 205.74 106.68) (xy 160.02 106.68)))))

